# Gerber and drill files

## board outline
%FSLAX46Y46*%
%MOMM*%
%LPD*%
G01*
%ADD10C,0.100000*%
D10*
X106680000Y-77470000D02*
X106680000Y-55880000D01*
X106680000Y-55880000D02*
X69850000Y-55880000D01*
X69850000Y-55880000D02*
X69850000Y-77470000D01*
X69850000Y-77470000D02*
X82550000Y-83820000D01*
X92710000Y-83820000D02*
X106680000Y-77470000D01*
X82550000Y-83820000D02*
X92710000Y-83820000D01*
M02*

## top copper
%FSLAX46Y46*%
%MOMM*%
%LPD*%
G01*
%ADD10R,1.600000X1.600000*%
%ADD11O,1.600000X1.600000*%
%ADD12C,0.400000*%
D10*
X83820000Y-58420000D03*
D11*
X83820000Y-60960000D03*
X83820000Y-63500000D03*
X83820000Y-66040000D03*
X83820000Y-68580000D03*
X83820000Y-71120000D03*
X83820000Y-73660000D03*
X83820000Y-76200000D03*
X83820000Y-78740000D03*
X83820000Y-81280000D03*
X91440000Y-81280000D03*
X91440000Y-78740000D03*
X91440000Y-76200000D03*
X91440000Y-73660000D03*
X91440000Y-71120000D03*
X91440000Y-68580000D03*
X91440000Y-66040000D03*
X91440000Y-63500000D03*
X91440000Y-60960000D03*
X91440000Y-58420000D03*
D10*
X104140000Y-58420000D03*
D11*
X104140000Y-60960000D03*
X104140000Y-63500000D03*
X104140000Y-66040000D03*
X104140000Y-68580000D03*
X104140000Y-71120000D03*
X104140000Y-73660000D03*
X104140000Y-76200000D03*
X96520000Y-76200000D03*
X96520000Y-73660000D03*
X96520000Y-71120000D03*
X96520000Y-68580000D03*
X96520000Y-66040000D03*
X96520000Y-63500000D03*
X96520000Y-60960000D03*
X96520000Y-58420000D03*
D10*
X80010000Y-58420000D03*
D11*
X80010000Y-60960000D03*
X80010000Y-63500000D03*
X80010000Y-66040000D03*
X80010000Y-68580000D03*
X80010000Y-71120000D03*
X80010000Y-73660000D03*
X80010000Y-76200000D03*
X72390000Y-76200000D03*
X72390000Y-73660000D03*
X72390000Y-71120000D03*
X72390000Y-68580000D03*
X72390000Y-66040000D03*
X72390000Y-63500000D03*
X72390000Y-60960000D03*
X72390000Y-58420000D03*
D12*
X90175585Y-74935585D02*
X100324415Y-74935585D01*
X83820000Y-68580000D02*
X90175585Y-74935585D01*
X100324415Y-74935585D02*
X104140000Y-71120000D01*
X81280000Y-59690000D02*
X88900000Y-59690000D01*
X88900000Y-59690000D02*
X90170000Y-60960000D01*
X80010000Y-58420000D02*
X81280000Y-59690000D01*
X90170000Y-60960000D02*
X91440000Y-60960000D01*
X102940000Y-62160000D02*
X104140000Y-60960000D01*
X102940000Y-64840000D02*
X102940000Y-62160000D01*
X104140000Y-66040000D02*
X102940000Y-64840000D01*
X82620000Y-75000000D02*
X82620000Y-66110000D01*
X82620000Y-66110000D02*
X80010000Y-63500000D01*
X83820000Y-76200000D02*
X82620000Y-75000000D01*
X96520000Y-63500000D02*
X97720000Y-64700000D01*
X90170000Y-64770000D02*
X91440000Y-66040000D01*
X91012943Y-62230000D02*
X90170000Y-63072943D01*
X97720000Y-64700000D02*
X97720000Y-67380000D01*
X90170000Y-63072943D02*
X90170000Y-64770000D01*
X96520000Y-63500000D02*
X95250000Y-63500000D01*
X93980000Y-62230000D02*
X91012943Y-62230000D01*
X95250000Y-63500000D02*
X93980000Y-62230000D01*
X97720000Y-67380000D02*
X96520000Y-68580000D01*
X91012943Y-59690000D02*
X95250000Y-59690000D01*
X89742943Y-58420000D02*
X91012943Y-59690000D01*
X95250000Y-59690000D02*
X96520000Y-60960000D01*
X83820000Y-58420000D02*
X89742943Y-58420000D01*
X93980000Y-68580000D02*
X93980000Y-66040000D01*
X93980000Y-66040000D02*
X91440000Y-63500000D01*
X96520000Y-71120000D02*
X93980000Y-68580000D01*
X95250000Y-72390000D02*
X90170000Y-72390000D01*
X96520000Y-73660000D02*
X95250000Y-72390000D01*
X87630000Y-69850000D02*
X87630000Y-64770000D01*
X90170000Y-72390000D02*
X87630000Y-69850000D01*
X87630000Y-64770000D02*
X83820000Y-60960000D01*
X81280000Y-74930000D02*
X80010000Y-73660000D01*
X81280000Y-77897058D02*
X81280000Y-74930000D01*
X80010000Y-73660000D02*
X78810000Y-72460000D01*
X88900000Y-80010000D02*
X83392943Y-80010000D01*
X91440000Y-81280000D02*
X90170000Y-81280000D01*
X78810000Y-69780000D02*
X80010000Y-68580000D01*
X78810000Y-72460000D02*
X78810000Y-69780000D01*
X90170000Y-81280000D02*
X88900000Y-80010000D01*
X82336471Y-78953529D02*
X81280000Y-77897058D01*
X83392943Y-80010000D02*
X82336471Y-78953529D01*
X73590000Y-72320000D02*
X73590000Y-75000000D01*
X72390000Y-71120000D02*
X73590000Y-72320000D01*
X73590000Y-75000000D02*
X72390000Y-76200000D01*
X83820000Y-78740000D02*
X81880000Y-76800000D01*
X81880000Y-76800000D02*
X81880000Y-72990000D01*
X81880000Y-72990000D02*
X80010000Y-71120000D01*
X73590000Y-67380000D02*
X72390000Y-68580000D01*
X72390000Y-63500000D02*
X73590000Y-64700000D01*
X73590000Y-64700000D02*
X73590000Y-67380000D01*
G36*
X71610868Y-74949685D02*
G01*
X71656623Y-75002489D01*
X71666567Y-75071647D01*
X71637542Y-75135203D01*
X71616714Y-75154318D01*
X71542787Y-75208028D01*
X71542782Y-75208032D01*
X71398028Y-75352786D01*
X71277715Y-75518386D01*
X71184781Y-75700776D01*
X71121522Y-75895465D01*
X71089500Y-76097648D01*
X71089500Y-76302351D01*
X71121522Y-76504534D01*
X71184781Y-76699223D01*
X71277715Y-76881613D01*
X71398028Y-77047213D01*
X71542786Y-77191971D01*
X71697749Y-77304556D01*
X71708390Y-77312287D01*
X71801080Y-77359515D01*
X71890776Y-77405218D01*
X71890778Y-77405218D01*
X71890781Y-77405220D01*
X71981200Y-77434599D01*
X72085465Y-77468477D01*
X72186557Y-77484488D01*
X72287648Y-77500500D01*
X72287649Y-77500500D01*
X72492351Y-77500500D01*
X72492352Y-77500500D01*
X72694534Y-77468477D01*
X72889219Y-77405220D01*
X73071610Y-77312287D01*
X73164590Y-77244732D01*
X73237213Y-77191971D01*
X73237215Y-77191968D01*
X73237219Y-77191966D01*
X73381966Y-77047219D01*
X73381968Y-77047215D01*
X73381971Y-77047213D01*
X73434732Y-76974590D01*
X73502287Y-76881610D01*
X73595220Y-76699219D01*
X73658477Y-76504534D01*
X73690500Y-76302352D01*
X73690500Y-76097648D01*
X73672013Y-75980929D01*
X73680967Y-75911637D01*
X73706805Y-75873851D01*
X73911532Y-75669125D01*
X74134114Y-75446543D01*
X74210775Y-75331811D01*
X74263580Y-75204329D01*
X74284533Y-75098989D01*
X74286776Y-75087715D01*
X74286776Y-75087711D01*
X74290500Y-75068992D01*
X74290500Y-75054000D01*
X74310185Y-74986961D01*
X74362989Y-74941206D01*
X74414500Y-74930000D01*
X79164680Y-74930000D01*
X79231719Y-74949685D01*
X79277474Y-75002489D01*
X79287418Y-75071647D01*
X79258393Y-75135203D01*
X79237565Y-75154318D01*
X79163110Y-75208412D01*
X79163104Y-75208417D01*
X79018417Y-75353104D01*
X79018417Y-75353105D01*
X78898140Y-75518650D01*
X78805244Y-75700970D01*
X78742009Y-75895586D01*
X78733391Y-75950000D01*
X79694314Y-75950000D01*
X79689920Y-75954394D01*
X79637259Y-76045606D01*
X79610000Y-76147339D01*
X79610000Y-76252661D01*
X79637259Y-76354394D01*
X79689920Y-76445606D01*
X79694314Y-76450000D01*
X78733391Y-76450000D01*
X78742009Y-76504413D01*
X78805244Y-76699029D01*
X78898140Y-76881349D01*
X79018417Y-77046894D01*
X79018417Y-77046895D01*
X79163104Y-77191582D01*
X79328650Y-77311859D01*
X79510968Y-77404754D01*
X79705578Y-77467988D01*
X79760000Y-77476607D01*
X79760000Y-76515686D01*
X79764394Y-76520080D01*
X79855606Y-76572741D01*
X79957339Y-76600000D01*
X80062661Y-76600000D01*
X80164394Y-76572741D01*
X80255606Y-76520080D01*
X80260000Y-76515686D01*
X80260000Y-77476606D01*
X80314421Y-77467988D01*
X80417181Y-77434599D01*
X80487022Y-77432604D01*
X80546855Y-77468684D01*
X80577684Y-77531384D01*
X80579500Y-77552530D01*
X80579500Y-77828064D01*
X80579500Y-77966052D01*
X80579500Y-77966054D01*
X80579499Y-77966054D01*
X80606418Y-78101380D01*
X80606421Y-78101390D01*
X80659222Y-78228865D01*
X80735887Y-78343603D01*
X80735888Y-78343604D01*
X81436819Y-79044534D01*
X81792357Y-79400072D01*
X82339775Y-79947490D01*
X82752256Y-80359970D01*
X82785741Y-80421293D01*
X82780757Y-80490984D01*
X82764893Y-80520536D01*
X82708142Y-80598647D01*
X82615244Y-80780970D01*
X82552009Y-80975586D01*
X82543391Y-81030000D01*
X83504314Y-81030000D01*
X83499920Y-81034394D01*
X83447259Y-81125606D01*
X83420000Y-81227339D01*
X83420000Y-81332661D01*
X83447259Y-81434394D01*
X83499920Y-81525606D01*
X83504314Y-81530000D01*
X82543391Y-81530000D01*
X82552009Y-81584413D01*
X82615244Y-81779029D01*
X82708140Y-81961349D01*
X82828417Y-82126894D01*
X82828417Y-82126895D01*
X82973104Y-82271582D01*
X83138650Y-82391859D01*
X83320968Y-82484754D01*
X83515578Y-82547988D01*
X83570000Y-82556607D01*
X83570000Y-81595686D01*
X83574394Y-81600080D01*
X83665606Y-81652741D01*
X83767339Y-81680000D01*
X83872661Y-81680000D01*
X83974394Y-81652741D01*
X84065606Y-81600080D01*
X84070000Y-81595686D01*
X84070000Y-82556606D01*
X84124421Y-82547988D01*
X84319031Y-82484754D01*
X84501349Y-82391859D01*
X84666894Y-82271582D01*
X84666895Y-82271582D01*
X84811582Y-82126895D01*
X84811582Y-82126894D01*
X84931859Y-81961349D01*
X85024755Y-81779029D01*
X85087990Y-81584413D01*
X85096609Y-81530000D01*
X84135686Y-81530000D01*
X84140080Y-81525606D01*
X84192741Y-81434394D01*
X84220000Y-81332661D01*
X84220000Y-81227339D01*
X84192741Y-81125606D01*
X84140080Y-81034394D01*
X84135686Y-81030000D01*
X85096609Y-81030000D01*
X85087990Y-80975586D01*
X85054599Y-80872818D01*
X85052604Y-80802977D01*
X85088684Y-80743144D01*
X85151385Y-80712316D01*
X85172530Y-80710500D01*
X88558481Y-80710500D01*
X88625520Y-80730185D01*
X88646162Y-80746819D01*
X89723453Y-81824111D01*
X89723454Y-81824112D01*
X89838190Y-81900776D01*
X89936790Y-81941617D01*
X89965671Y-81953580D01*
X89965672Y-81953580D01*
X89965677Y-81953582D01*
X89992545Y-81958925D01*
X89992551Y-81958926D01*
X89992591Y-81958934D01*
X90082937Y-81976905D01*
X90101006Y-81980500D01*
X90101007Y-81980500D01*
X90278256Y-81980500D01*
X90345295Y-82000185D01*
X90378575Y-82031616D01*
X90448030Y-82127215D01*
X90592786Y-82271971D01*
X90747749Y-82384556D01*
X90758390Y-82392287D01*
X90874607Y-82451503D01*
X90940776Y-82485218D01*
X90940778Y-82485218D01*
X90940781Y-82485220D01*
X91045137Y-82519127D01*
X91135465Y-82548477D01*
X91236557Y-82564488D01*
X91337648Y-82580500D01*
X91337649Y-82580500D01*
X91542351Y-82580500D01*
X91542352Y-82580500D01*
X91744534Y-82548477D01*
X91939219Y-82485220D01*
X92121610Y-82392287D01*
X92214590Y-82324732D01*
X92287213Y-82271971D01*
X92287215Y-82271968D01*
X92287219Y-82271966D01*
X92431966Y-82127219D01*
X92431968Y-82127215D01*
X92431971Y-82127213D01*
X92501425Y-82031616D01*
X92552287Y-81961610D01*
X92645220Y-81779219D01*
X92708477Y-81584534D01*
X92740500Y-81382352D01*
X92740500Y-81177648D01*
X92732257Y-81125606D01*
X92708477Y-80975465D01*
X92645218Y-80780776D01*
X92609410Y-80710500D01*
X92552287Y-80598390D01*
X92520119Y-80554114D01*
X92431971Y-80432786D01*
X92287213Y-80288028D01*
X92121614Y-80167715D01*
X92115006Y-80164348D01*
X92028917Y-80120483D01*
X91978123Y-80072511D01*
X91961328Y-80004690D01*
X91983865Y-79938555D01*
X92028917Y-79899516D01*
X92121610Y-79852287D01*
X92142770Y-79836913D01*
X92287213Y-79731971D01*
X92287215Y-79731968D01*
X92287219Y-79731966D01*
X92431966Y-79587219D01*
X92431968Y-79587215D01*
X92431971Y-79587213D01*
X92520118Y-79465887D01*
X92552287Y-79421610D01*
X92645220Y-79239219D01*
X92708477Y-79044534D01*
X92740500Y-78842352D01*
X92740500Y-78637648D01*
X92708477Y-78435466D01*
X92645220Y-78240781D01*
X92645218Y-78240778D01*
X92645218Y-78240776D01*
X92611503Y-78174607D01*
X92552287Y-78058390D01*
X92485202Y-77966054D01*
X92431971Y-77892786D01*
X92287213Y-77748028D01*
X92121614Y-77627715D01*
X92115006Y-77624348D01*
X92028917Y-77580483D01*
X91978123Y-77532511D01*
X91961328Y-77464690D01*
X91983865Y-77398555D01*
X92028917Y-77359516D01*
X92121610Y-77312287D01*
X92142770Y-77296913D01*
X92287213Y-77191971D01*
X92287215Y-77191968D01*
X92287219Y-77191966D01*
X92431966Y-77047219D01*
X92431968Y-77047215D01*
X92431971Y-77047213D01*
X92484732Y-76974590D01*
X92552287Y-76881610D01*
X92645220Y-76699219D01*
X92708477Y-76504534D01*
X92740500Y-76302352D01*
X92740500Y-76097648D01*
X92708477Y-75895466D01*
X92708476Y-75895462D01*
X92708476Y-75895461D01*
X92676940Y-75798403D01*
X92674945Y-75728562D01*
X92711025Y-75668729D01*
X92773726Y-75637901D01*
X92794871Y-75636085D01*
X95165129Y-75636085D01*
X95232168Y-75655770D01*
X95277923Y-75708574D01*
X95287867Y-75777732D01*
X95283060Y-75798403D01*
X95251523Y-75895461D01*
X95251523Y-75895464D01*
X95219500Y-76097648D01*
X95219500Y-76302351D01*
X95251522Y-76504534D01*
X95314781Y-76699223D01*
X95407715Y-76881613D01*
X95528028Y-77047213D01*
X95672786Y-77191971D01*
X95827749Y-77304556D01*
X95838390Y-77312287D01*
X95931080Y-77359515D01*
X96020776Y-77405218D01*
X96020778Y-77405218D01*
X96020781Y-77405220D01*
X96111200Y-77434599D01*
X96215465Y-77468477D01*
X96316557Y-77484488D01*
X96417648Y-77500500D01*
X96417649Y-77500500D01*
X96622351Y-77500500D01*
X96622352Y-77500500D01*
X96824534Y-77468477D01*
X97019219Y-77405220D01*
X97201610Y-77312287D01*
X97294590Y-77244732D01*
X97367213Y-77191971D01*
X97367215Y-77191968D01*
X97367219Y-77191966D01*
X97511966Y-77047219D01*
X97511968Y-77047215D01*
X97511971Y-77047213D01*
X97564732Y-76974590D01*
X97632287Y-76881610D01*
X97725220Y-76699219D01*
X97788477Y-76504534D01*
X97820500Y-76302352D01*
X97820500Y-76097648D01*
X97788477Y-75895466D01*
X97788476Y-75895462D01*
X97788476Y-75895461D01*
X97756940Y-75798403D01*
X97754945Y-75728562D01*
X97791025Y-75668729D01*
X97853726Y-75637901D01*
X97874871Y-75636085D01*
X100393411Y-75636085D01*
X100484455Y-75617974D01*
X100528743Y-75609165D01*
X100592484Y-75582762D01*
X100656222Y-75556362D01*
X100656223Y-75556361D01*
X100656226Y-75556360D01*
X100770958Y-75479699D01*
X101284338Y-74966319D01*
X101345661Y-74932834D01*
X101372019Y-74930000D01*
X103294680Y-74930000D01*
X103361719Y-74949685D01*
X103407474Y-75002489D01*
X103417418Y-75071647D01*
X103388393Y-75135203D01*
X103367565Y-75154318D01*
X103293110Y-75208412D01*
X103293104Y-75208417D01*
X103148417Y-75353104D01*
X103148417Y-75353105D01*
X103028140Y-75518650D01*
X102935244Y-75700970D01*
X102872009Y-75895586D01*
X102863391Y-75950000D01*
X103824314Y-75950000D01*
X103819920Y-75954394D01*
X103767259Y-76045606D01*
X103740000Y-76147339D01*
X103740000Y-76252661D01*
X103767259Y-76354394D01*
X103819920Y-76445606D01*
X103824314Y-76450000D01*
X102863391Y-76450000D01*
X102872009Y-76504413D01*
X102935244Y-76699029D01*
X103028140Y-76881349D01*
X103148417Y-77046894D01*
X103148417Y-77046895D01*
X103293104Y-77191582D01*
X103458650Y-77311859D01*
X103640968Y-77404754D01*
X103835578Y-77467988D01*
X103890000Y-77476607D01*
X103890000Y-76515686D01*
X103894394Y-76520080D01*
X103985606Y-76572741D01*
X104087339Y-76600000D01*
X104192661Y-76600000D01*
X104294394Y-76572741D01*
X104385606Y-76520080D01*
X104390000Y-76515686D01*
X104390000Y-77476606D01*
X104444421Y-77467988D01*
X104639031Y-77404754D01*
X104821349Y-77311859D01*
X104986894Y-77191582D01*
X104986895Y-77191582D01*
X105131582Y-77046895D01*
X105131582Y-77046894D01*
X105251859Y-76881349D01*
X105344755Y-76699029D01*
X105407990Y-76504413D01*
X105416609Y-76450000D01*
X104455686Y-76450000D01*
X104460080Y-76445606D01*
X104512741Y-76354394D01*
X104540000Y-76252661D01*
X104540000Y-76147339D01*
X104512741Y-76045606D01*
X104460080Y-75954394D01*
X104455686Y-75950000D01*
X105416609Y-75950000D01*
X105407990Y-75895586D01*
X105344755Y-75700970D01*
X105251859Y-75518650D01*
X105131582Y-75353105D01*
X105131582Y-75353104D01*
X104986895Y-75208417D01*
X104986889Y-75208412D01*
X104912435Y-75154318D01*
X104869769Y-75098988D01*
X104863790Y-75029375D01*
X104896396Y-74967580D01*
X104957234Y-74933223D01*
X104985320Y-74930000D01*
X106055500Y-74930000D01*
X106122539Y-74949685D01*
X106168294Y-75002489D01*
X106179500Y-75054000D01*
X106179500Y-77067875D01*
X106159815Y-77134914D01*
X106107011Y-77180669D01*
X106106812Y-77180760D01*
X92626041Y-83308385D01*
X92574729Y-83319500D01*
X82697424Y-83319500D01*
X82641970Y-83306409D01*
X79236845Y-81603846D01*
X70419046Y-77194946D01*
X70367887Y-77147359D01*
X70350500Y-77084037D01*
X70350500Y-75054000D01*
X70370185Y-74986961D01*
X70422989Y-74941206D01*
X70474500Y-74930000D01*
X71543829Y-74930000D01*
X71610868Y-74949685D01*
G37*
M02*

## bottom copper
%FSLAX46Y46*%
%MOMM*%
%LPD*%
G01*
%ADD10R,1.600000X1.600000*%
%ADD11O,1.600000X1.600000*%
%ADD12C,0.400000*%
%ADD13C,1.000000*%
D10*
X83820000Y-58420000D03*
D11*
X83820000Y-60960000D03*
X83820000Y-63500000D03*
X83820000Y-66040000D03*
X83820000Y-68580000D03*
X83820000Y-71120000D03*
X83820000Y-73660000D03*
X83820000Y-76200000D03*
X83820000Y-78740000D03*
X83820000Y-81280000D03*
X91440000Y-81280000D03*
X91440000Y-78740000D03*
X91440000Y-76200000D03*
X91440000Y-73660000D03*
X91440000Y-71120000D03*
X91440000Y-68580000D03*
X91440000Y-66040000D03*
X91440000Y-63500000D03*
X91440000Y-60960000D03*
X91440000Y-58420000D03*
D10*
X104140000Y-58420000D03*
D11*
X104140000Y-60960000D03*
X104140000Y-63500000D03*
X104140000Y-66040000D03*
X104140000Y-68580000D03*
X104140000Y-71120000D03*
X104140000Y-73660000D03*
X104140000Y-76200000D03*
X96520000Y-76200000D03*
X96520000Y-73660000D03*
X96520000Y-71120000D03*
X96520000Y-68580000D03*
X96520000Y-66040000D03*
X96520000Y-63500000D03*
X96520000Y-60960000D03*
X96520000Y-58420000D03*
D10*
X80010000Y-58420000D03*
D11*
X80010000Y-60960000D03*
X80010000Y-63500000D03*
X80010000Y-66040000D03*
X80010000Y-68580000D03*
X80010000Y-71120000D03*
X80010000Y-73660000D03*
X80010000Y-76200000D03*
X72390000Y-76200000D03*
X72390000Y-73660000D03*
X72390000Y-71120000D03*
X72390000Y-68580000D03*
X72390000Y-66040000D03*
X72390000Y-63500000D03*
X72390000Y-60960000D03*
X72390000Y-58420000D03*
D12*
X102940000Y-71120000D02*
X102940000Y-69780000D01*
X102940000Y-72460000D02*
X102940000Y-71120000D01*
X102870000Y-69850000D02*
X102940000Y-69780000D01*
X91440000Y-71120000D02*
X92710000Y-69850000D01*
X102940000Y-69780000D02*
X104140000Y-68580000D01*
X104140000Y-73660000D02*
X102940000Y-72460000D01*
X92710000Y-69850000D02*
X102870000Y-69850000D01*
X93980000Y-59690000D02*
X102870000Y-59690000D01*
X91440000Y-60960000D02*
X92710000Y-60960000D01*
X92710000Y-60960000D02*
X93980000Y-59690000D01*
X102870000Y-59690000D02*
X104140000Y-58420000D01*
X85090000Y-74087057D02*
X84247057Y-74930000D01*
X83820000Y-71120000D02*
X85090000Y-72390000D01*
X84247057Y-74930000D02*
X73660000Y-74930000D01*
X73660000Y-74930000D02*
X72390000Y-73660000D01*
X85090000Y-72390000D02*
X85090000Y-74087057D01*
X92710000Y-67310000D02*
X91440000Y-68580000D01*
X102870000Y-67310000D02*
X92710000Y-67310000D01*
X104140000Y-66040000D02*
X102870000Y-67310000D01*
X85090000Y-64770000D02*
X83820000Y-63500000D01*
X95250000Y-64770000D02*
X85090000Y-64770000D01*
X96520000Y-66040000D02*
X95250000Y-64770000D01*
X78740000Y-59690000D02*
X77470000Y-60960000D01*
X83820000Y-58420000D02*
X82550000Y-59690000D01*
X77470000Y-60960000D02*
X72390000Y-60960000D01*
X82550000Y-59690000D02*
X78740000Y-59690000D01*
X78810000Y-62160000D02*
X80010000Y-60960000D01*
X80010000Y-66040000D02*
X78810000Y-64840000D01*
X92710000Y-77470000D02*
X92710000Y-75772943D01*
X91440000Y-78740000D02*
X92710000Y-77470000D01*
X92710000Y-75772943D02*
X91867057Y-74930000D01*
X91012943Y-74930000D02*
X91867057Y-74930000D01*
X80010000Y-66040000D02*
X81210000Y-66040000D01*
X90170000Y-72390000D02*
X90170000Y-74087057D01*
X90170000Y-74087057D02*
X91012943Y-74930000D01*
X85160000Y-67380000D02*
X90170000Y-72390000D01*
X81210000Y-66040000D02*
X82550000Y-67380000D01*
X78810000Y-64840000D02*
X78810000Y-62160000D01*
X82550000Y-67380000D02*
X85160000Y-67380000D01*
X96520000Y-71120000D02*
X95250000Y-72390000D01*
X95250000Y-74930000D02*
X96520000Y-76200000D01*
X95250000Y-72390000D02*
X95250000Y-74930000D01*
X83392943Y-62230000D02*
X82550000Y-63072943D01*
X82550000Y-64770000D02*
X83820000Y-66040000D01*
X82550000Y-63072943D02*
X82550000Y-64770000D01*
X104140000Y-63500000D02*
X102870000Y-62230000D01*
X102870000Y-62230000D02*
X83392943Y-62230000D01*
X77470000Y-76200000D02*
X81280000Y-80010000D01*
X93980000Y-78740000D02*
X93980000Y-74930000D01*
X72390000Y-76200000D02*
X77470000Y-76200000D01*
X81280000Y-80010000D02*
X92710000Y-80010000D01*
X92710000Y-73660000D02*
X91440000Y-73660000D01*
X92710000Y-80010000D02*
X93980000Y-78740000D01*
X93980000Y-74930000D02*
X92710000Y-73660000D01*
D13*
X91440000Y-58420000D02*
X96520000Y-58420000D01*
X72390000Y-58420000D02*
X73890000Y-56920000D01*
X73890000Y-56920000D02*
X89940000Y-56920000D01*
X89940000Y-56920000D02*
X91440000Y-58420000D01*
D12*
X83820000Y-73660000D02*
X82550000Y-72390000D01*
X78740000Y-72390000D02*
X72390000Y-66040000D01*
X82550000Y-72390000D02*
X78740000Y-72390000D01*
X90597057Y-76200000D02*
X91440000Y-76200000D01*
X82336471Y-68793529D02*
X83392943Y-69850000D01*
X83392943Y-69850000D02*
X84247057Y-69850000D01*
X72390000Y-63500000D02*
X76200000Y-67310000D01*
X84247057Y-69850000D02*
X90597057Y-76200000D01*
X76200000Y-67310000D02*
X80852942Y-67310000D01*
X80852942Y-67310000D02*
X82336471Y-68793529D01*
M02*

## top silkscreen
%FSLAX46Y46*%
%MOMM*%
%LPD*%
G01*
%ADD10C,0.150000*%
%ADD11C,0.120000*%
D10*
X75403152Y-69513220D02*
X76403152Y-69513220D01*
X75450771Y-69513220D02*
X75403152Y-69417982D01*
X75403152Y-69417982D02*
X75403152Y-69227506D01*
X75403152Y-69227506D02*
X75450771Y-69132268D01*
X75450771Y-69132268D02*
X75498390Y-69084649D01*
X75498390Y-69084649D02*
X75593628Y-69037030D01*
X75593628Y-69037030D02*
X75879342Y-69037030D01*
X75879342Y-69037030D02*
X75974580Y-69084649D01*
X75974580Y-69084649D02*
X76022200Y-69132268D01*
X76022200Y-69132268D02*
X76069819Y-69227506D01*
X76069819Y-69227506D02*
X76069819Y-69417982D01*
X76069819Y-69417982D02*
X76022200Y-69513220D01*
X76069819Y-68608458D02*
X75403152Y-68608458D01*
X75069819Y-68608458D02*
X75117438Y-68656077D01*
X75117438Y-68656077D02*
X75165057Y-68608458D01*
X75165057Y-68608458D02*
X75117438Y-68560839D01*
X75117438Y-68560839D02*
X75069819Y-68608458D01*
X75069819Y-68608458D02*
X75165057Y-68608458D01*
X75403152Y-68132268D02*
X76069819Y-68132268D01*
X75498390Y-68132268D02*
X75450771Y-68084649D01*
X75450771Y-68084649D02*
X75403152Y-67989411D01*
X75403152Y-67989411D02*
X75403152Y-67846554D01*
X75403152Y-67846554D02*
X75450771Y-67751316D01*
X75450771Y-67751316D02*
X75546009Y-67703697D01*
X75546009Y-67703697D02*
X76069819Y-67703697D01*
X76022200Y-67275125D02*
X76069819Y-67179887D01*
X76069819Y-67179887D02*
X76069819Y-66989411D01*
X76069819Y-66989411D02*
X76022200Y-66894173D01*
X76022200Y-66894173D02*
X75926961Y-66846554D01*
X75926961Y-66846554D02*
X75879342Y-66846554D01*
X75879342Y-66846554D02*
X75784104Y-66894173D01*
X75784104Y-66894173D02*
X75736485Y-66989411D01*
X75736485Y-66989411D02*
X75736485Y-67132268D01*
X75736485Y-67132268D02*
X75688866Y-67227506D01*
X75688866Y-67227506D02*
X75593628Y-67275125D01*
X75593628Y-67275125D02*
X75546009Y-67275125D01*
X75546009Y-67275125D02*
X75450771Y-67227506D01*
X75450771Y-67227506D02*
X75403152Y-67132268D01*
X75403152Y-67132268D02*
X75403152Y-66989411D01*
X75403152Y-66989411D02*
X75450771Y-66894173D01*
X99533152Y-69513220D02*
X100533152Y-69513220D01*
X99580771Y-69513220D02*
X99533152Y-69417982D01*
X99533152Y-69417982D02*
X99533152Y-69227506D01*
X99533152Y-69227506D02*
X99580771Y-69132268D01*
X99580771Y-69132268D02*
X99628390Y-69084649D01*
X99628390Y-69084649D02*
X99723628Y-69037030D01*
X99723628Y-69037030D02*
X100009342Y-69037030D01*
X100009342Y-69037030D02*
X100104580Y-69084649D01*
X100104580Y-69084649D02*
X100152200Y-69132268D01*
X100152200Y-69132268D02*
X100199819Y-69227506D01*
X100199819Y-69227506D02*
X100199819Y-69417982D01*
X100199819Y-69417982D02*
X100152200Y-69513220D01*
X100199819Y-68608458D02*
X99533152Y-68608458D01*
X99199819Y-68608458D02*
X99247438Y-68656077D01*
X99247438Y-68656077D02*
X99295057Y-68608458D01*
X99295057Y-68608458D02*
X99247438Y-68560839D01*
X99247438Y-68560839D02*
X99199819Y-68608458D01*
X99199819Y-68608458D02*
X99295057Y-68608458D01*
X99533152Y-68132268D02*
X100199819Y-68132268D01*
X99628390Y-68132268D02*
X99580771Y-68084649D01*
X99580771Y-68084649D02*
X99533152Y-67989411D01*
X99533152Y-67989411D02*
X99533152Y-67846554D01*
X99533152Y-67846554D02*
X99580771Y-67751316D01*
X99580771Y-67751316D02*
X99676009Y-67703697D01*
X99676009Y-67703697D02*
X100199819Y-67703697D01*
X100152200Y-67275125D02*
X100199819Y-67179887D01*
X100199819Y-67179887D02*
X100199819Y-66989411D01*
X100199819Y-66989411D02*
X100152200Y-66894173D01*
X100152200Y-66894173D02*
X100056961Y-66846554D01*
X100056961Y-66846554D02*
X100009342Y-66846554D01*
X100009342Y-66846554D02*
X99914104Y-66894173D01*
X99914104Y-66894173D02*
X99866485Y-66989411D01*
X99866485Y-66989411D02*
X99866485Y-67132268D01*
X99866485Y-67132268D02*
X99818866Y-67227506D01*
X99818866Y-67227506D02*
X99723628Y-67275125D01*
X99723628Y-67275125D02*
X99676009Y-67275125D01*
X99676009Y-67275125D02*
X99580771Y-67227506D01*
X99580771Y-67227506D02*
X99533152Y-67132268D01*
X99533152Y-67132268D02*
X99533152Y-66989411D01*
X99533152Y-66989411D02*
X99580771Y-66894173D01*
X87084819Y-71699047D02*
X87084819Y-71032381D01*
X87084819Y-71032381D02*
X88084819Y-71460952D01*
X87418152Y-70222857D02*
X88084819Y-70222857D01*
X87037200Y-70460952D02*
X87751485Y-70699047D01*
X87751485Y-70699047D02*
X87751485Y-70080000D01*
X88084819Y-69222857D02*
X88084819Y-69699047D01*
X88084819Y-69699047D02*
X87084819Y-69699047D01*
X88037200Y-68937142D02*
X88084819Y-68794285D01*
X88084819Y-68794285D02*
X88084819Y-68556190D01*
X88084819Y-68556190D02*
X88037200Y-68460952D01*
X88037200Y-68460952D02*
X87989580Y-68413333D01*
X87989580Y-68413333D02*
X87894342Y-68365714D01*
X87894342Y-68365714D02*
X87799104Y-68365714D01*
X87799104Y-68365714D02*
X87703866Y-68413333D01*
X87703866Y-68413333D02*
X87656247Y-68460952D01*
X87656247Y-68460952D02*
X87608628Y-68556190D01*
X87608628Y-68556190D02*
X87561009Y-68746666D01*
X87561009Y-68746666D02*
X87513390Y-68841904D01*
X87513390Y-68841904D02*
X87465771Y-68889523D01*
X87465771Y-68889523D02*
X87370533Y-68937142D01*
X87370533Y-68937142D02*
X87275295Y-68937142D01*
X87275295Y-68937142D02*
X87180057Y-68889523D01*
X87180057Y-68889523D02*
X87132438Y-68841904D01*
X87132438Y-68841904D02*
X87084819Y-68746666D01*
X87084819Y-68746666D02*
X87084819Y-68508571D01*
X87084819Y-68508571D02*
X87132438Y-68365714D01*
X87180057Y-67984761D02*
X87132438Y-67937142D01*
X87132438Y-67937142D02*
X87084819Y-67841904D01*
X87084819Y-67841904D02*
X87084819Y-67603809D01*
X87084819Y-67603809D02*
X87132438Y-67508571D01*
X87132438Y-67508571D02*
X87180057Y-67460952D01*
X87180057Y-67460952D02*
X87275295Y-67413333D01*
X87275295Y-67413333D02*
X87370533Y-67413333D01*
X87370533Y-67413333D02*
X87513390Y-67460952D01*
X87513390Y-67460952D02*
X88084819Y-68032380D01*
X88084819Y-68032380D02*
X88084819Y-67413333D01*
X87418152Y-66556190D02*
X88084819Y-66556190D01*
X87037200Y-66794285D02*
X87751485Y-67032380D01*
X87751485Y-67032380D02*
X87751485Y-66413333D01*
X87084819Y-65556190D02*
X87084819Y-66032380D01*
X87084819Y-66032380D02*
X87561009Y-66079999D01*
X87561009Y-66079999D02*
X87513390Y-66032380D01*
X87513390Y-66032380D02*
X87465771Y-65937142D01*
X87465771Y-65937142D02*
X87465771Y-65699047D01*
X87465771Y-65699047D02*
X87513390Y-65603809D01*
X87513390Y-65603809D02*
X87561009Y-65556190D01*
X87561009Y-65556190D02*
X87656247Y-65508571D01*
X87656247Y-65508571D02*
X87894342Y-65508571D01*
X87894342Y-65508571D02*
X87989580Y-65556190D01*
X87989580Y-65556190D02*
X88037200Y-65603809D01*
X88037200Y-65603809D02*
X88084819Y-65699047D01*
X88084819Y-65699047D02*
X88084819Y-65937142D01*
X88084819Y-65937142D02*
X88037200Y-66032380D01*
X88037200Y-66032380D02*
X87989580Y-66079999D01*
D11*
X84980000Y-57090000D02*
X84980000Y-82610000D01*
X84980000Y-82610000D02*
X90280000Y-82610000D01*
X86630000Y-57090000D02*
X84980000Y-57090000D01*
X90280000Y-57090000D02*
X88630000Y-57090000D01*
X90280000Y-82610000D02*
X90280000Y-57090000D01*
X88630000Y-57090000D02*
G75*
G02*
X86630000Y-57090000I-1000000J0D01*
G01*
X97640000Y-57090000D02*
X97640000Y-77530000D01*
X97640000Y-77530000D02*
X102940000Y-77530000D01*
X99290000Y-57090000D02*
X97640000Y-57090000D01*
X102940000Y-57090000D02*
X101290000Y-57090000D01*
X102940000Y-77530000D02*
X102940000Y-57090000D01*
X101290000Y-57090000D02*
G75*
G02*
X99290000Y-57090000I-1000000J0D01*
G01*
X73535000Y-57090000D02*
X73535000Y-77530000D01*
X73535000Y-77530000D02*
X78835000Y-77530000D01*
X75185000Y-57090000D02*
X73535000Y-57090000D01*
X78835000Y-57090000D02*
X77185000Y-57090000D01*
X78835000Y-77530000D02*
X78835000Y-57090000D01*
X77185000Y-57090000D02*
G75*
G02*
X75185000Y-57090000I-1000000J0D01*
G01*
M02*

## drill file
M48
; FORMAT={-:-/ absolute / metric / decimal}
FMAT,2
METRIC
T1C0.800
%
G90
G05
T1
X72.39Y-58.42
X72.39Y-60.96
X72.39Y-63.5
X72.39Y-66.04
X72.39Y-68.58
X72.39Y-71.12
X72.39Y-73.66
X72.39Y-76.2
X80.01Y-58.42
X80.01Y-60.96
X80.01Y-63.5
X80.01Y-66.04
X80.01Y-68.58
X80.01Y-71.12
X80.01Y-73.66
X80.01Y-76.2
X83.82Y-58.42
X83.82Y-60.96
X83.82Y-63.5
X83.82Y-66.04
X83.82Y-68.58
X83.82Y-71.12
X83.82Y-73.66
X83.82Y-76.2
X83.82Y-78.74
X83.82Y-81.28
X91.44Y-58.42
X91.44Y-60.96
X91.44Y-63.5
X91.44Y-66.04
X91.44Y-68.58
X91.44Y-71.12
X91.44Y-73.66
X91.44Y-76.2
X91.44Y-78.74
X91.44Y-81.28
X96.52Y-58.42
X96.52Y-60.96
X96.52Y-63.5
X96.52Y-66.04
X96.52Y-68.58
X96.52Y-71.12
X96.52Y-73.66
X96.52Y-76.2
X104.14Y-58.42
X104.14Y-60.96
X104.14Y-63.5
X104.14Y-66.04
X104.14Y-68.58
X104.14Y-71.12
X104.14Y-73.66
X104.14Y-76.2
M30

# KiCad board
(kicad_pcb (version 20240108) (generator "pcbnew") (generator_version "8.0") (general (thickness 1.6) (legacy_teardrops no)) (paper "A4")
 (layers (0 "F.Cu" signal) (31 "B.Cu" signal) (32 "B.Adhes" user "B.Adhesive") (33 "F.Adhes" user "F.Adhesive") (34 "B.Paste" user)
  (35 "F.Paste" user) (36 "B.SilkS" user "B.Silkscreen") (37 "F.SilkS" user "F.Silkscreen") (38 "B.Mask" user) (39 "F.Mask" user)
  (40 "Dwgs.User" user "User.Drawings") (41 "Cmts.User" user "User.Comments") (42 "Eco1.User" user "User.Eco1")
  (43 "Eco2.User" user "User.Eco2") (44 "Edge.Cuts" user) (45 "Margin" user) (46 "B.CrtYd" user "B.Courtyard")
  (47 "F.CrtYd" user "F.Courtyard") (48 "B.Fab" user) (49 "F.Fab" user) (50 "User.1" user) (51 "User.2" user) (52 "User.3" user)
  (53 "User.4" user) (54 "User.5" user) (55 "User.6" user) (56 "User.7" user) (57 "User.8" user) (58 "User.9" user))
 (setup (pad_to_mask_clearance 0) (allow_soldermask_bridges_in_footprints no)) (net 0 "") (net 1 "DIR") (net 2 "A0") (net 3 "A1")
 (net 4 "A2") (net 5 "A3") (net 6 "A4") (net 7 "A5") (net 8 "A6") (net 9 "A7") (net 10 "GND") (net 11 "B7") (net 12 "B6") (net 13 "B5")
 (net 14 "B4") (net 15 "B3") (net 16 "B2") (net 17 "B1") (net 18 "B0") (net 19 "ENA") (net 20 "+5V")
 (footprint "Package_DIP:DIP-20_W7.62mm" (layer "F.Cu") (at 83.82 58.42)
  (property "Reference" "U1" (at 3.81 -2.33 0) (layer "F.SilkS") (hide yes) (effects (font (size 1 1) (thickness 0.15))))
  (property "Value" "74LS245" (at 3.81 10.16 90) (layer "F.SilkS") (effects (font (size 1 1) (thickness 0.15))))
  (fp_line (start 1.16 -1.33) (end 1.16 24.19) (stroke (width 0.12) (type solid)) (layer "F.SilkS"))
  (fp_line (start 1.16 24.19) (end 6.46 24.19) (stroke (width 0.12) (type solid)) (layer "F.SilkS"))
  (fp_line (start 2.81 -1.33) (end 1.16 -1.33) (stroke (width 0.12) (type solid)) (layer "F.SilkS"))
  (fp_line (start 6.46 -1.33) (end 4.81 -1.33) (stroke (width 0.12) (type solid)) (layer "F.SilkS"))
  (fp_line (start 6.46 24.19) (end 6.46 -1.33) (stroke (width 0.12) (type solid)) (layer "F.SilkS"))
  (fp_arc (start 4.81 -1.33) (mid 3.81 -0.33) (end 2.81 -1.33) (stroke (width 0.12) (type solid)) (layer "F.SilkS"))
  (pad "1" thru_hole rect (at 0 0) (size 1.6 1.6) (drill 0.8) (layers "*.Cu" "*.Mask") (remove_unused_layers no) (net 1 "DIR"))
  (pad "2" thru_hole oval (at 0 2.54) (size 1.6 1.6) (drill 0.8) (layers "*.Cu" "*.Mask") (remove_unused_layers no) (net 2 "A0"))
  (pad "3" thru_hole oval (at 0 5.08) (size 1.6 1.6) (drill 0.8) (layers "*.Cu" "*.Mask") (remove_unused_layers no) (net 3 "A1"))
  (pad "4" thru_hole oval (at 0 7.62) (size 1.6 1.6) (drill 0.8) (layers "*.Cu" "*.Mask") (remove_unused_layers no) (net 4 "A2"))
  (pad "5" thru_hole oval (at 0 10.16) (size 1.6 1.6) (drill 0.8) (layers "*.Cu" "*.Mask") (remove_unused_layers no) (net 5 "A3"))
  (pad "6" thru_hole oval (at 0 12.7) (size 1.6 1.6) (drill 0.8) (layers "*.Cu" "*.Mask") (remove_unused_layers no) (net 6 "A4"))
  (pad "7" thru_hole oval (at 0 15.24) (size 1.6 1.6) (drill 0.8) (layers "*.Cu" "*.Mask") (remove_unused_layers no) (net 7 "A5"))
  (pad "8" thru_hole oval (at 0 17.78) (size 1.6 1.6) (drill 0.8) (layers "*.Cu" "*.Mask") (remove_unused_layers no) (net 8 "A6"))
  (pad "9" thru_hole oval (at 0 20.32) (size 1.6 1.6) (drill 0.8) (layers "*.Cu" "*.Mask") (remove_unused_layers no) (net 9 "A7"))
  (pad "10" thru_hole oval (at 0 22.86) (size 1.6 1.6) (drill 0.8) (layers "*.Cu" "*.Mask") (remove_unused_layers no) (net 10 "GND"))
  (pad "11" thru_hole oval (at 7.62 22.86) (size 1.6 1.6) (drill 0.8) (layers "*.Cu" "*.Mask") (remove_unused_layers no) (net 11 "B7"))
  (pad "12" thru_hole oval (at 7.62 20.32) (size 1.6 1.6) (drill 0.8) (layers "*.Cu" "*.Mask") (remove_unused_layers no) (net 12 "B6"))
  (pad "13" thru_hole oval (at 7.62 17.78) (size 1.6 1.6) (drill 0.8) (layers "*.Cu" "*.Mask") (remove_unused_layers no) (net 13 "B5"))
  (pad "14" thru_hole oval (at 7.62 15.24) (size 1.6 1.6) (drill 0.8) (layers "*.Cu" "*.Mask") (remove_unused_layers no) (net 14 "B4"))
  (pad "15" thru_hole oval (at 7.62 12.7) (size 1.6 1.6) (drill 0.8) (layers "*.Cu" "*.Mask") (remove_unused_layers no) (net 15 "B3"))
  (pad "16" thru_hole oval (at 7.62 10.16) (size 1.6 1.6) (drill 0.8) (layers "*.Cu" "*.Mask") (remove_unused_layers no) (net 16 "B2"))
  (pad "17" thru_hole oval (at 7.62 7.62) (size 1.6 1.6) (drill 0.8) (layers "*.Cu" "*.Mask") (remove_unused_layers no) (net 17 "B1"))
  (pad "18" thru_hole oval (at 7.62 5.08) (size 1.6 1.6) (drill 0.8) (layers "*.Cu" "*.Mask") (remove_unused_layers no) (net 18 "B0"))
  (pad "19" thru_hole oval (at 7.62 2.54) (size 1.6 1.6) (drill 0.8) (layers "*.Cu" "*.Mask") (remove_unused_layers no) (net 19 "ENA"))
  (pad "20" thru_hole oval (at 7.62 0) (size 1.6 1.6) (drill 0.8) (layers "*.Cu" "*.Mask") (remove_unused_layers no) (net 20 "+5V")))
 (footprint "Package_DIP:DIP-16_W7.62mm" (layer "B.Cu") (at 104.14 58.42 180)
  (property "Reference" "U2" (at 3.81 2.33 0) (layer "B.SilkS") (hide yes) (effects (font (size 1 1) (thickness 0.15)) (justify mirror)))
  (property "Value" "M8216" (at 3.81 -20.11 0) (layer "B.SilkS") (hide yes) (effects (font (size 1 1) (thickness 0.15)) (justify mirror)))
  (fp_line (start 6.5 1.33) (end 6.5 -19.11) (stroke (width 0.12) (type solid)) (layer "F.SilkS"))
  (fp_line (start 6.5 -19.11) (end 1.2 -19.11) (stroke (width 0.12) (type solid)) (layer "F.SilkS"))
  (fp_line (start 4.85 1.33) (end 6.5 1.33) (stroke (width 0.12) (type solid)) (layer "F.SilkS"))
  (fp_line (start 1.2 1.33) (end 2.85 1.33) (stroke (width 0.12) (type solid)) (layer "F.SilkS"))
  (fp_line (start 1.2 -19.11) (end 1.2 1.33) (stroke (width 0.12) (type solid)) (layer "F.SilkS"))
  (fp_arc (start 2.85 1.33) (mid 3.85 0.33) (end 4.85 1.33) (stroke (width 0.12) (type solid)) (layer "F.SilkS"))
  (pad "1" thru_hole rect (at 0 0 180) (size 1.6 1.6) (drill 0.8) (layers "*.Cu" "*.Mask") (remove_unused_layers no) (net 19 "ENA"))
  (pad "2" thru_hole oval (at 0 -2.54 180) (size 1.6 1.6) (drill 0.8) (layers "*.Cu" "*.Mask") (remove_unused_layers no) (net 16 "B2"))
  (pad "3" thru_hole oval (at 0 -5.08 180) (size 1.6 1.6) (drill 0.8) (layers "*.Cu" "*.Mask") (remove_unused_layers no) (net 4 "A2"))
  (pad "4" thru_hole oval (at 0 -7.62 180) (size 1.6 1.6) (drill 0.8) (layers "*.Cu" "*.Mask") (remove_unused_layers no) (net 16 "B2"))
  (pad "5" thru_hole oval (at 0 -10.16 180) (size 1.6 1.6) (drill 0.8) (layers "*.Cu" "*.Mask") (remove_unused_layers no) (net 15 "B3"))
  (pad "6" thru_hole oval (at 0 -12.7 180) (size 1.6 1.6) (drill 0.8) (layers "*.Cu" "*.Mask") (remove_unused_layers no) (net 5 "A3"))
  (pad "7" thru_hole oval (at 0 -15.24 180) (size 1.6 1.6) (drill 0.8) (layers "*.Cu" "*.Mask") (remove_unused_layers no) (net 15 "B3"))
  (pad "8" thru_hole oval (at 0 -17.78 180) (size 1.6 1.6) (drill 0.8) (layers "*.Cu" "*.Mask") (remove_unused_layers no) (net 10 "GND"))
  (pad "9" thru_hole oval (at 7.62 -17.78 180) (size 1.6 1.6) (drill 0.8) (layers "*.Cu" "*.Mask") (remove_unused_layers no) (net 18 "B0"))
  (pad "10" thru_hole oval (at 7.62 -15.24 180) (size 1.6 1.6) (drill 0.8) (layers "*.Cu" "*.Mask") (remove_unused_layers no) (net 2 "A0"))
  (pad "11" thru_hole oval (at 7.62 -12.7 180) (size 1.6 1.6) (drill 0.8) (layers "*.Cu" "*.Mask") (remove_unused_layers no) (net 18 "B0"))
  (pad "12" thru_hole oval (at 7.62 -10.16 180) (size 1.6 1.6) (drill 0.8) (layers "*.Cu" "*.Mask") (remove_unused_layers no) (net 17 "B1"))
  (pad "13" thru_hole oval (at 7.62 -7.62 180) (size 1.6 1.6) (drill 0.8) (layers "*.Cu" "*.Mask") (remove_unused_layers no) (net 3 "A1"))
  (pad "14" thru_hole oval (at 7.62 -5.08 180) (size 1.6 1.6) (drill 0.8) (layers "*.Cu" "*.Mask") (remove_unused_layers no) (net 17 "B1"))
  (pad "15" thru_hole oval (at 7.62 -2.54 180) (size 1.6 1.6) (drill 0.8) (layers "*.Cu" "*.Mask") (remove_unused_layers no) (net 1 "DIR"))
  (pad "16" thru_hole oval (at 7.62 0 180) (size 1.6 1.6) (drill 0.8) (layers "*.Cu" "*.Mask") (remove_unused_layers no) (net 20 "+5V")))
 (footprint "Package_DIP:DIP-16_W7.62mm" (layer "B.Cu") (at 80.01 58.42 180)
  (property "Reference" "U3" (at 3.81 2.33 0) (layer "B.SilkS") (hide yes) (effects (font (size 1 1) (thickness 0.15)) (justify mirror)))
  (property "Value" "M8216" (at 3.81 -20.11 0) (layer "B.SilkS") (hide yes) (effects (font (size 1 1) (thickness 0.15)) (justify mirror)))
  (fp_line (start 6.475 1.33) (end 6.475 -19.11) (stroke (width 0.12) (type solid)) (layer "F.SilkS"))
  (fp_line (start 6.475 -19.11) (end 1.175 -19.11) (stroke (width 0.12) (type solid)) (layer "F.SilkS"))
  (fp_line (start 4.825 1.33) (end 6.475 1.33) (stroke (width 0.12) (type solid)) (layer "F.SilkS"))
  (fp_line (start 1.175 1.33) (end 2.825 1.33) (stroke (width 0.12) (type solid)) (layer "F.SilkS"))
  (fp_line (start 1.175 -19.11) (end 1.175 1.33) (stroke (width 0.12) (type solid)) (layer "F.SilkS"))
  (fp_arc (start 2.825 1.33) (mid 3.825 0.33) (end 4.825 1.33) (stroke (width 0.12) (type solid)) (layer "F.SilkS"))
  (pad "1" thru_hole rect (at 0 0 180) (size 1.6 1.6) (drill 0.8) (layers "*.Cu" "*.Mask") (remove_unused_layers no) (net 19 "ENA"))
  (pad "2" thru_hole oval (at 0 -2.54 180) (size 1.6 1.6) (drill 0.8) (layers "*.Cu" "*.Mask") (remove_unused_layers no) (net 12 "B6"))
  (pad "3" thru_hole oval (at 0 -5.08 180) (size 1.6 1.6) (drill 0.8) (layers "*.Cu" "*.Mask") (remove_unused_layers no) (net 8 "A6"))
  (pad "4" thru_hole oval (at 0 -7.62 180) (size 1.6 1.6) (drill 0.8) (layers "*.Cu" "*.Mask") (remove_unused_layers no) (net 12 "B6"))
  (pad "5" thru_hole oval (at 0 -10.16 180) (size 1.6 1.6) (drill 0.8) (layers "*.Cu" "*.Mask") (remove_unused_layers no) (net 11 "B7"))
  (pad "6" thru_hole oval (at 0 -12.7 180) (size 1.6 1.6) (drill 0.8) (layers "*.Cu" "*.Mask") (remove_unused_layers no) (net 9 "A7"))
  (pad "7" thru_hole oval (at 0 -15.24 180) (size 1.6 1.6) (drill 0.8) (layers "*.Cu" "*.Mask") (remove_unused_layers no) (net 11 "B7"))
  (pad "8" thru_hole oval (at 0 -17.78 180) (size 1.6 1.6) (drill 0.8) (layers "*.Cu" "*.Mask") (remove_unused_layers no) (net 10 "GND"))
  (pad "9" thru_hole oval (at 7.62 -17.78 180) (size 1.6 1.6) (drill 0.8) (layers "*.Cu" "*.Mask") (remove_unused_layers no) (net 14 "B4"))
  (pad "10" thru_hole oval (at 7.62 -15.24 180) (size 1.6 1.6) (drill 0.8) (layers "*.Cu" "*.Mask") (remove_unused_layers no) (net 6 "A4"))
  (pad "11" thru_hole oval (at 7.62 -12.7 180) (size 1.6 1.6) (drill 0.8) (layers "*.Cu" "*.Mask") (remove_unused_layers no) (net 14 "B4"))
  (pad "12" thru_hole oval (at 7.62 -10.16 180) (size 1.6 1.6) (drill 0.8) (layers "*.Cu" "*.Mask") (remove_unused_layers no) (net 13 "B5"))
  (pad "13" thru_hole oval (at 7.62 -7.62 180) (size 1.6 1.6) (drill 0.8) (layers "*.Cu" "*.Mask") (remove_unused_layers no) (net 7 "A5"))
  (pad "14" thru_hole oval (at 7.62 -5.08 180) (size 1.6 1.6) (drill 0.8) (layers "*.Cu" "*.Mask") (remove_unused_layers no) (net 13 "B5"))
  (pad "15" thru_hole oval (at 7.62 -2.54 180) (size 1.6 1.6) (drill 0.8) (layers "*.Cu" "*.Mask") (remove_unused_layers no) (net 1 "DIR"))
  (pad "16" thru_hole oval (at 7.62 0 180) (size 1.6 1.6) (drill 0.8) (layers "*.Cu" "*.Mask") (remove_unused_layers no) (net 20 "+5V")))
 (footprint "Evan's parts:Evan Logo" (layer "B.Cu") (at 87.63 59.69 -90)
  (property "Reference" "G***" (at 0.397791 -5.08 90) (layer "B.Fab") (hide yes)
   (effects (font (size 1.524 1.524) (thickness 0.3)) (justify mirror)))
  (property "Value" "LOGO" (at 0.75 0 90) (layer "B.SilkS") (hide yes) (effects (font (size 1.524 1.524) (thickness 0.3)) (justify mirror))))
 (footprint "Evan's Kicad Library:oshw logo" (layer "B.Cu") (at 100.33 67.31 -90)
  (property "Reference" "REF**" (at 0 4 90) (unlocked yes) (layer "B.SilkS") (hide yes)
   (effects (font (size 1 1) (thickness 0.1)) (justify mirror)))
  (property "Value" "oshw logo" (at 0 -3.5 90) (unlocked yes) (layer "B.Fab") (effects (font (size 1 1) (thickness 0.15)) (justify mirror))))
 (gr_line (start 106.68 77.47) (end 106.68 55.88) (stroke (width 0.1) (type default)) (layer "Edge.Cuts"))
 (gr_line (start 106.68 55.88) (end 69.85 55.88) (stroke (width 0.1) (type default)) (layer "Edge.Cuts"))
 (gr_line (start 69.85 55.88) (end 69.85 77.47) (stroke (width 0.1) (type default)) (layer "Edge.Cuts"))
 (gr_line (start 69.85 77.47) (end 82.55 83.82) (stroke (width 0.1) (type default)) (layer "Edge.Cuts"))
 (gr_line (start 92.71 83.82) (end 106.68 77.47) (stroke (width 0.1) (type default)) (layer "Edge.Cuts"))
 (gr_line (start 82.55 83.82) (end 92.71 83.82) (stroke (width 0.1) (type default)) (layer "Edge.Cuts"))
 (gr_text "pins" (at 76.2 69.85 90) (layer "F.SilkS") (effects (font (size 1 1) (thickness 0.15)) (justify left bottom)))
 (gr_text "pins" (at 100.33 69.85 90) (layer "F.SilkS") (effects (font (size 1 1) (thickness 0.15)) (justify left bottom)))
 (segment (start 90.175585 74.935585) (end 100.324415 74.935585) (width 0.4) (layer "F.Cu") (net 5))
 (segment (start 83.82 68.58) (end 90.175585 74.935585) (width 0.4) (layer "F.Cu") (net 5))
 (segment (start 100.324415 74.935585) (end 104.14 71.12) (width 0.4) (layer "F.Cu") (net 5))
 (segment (start 102.94 71.12) (end 102.94 69.78) (width 0.4) (layer "B.Cu") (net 15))
 (segment (start 102.94 72.46) (end 102.94 71.12) (width 0.4) (layer "B.Cu") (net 15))
 (segment (start 102.87 69.85) (end 102.94 69.78) (width 0.4) (layer "B.Cu") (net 15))
 (segment (start 91.44 71.12) (end 92.71 69.85) (width 0.4) (layer "B.Cu") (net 15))
 (segment (start 102.94 69.78) (end 104.14 68.58) (width 0.4) (layer "B.Cu") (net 15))
 (segment (start 104.14 73.66) (end 102.94 72.46) (width 0.4) (layer "B.Cu") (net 15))
 (segment (start 92.71 69.85) (end 102.87 69.85) (width 0.4) (layer "B.Cu") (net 15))
 (segment (start 81.28 59.69) (end 88.9 59.69) (width 0.4) (layer "F.Cu") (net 19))
 (segment (start 88.9 59.69) (end 90.17 60.96) (width 0.4) (layer "F.Cu") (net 19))
 (segment (start 80.01 58.42) (end 81.28 59.69) (width 0.4) (layer "F.Cu") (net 19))
 (segment (start 90.17 60.96) (end 91.44 60.96) (width 0.4) (layer "F.Cu") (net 19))
 (segment (start 93.98 59.69) (end 102.87 59.69) (width 0.4) (layer "B.Cu") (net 19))
 (segment (start 91.44 60.96) (end 92.71 60.96) (width 0.4) (layer "B.Cu") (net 19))
 (segment (start 92.71 60.96) (end 93.98 59.69) (width 0.4) (layer "B.Cu") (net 19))
 (segment (start 102.87 59.69) (end 104.14 58.42) (width 0.4) (layer "B.Cu") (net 19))
 (segment (start 85.09 74.087057) (end 84.247057 74.93) (width 0.4) (layer "B.Cu") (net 6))
 (segment (start 83.82 71.12) (end 85.09 72.39) (width 0.4) (layer "B.Cu") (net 6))
 (segment (start 84.247057 74.93) (end 73.66 74.93) (width 0.4) (layer "B.Cu") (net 6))
 (segment (start 73.66 74.93) (end 72.39 73.66) (width 0.4) (layer "B.Cu") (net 6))
 (segment (start 85.09 72.39) (end 85.09 74.087057) (width 0.4) (layer "B.Cu") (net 6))
 (segment (start 102.94 62.16) (end 104.14 60.96) (width 0.4) (layer "F.Cu") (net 16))
 (segment (start 102.94 64.84) (end 102.94 62.16) (width 0.4) (layer "F.Cu") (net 16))
 (segment (start 104.14 66.04) (end 102.94 64.84) (width 0.4) (layer "F.Cu") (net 16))
 (segment (start 92.71 67.31) (end 91.44 68.58) (width 0.4) (layer "B.Cu") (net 16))
 (segment (start 102.87 67.31) (end 92.71 67.31) (width 0.4) (layer "B.Cu") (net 16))
 (segment (start 104.14 66.04) (end 102.87 67.31) (width 0.4) (layer "B.Cu") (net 16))
 (segment (start 82.62 75) (end 82.62 66.11) (width 0.4) (layer "F.Cu") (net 8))
 (segment (start 82.62 66.11) (end 80.01 63.5) (width 0.4) (layer "F.Cu") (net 8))
 (segment (start 83.82 76.2) (end 82.62 75) (width 0.4) (layer "F.Cu") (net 8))
 (segment (start 96.52 63.5) (end 97.72 64.7) (width 0.4) (layer "F.Cu") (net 17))
 (segment (start 90.17 64.77) (end 91.44 66.04) (width 0.4) (layer "F.Cu") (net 17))
 (segment (start 91.012943 62.23) (end 90.17 63.072943) (width 0.4) (layer "F.Cu") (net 17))
 (segment (start 97.72 64.7) (end 97.72 67.38) (width 0.4) (layer "F.Cu") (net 17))
 (segment (start 90.17 63.072943) (end 90.17 64.77) (width 0.4) (layer "F.Cu") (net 17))
 (segment (start 96.52 63.5) (end 95.25 63.5) (width 0.4) (layer "F.Cu") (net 17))
 (segment (start 93.98 62.23) (end 91.012943 62.23) (width 0.4) (layer "F.Cu") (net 17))
 (segment (start 95.25 63.5) (end 93.98 62.23) (width 0.4) (layer "F.Cu") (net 17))
 (segment (start 97.72 67.38) (end 96.52 68.58) (width 0.4) (layer "F.Cu") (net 17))
 (segment (start 85.09 64.77) (end 83.82 63.5) (width 0.4) (layer "B.Cu") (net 3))
 (segment (start 95.25 64.77) (end 85.09 64.77) (width 0.4) (layer "B.Cu") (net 3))
 (segment (start 96.52 66.04) (end 95.25 64.77) (width 0.4) (layer "B.Cu") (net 3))
 (segment (start 91.012943 59.69) (end 95.25 59.69) (width 0.4) (layer "F.Cu") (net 1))
 (segment (start 89.742943 58.42) (end 91.012943 59.69) (width 0.4) (layer "F.Cu") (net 1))
 (segment (start 95.25 59.69) (end 96.52 60.96) (width 0.4) (layer "F.Cu") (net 1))
 (segment (start 83.82 58.42) (end 89.742943 58.42) (width 0.4) (layer "F.Cu") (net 1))
 (segment (start 78.74 59.69) (end 77.47 60.96) (width 0.4) (layer "B.Cu") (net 1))
 (segment (start 83.82 58.42) (end 82.55 59.69) (width 0.4) (layer "B.Cu") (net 1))
 (segment (start 77.47 60.96) (end 72.39 60.96) (width 0.4) (layer "B.Cu") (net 1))
 (segment (start 82.55 59.69) (end 78.74 59.69) (width 0.4) (layer "B.Cu") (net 1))
 (segment (start 78.81 62.16) (end 80.01 60.96) (width 0.4) (layer "B.Cu") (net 12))
 (segment (start 80.01 66.04) (end 78.81 64.84) (width 0.4) (layer "B.Cu") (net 12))
 (segment (start 92.71 77.47) (end 92.71 75.772943) (width 0.4) (layer "B.Cu") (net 12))
 (segment (start 91.44 78.74) (end 92.71 77.47) (width 0.4) (layer "B.Cu") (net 12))
 (segment (start 92.71 75.772943) (end 91.867057 74.93) (width 0.4) (layer "B.Cu") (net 12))
 (segment (start 91.012943 74.93) (end 91.867057 74.93) (width 0.4) (layer "B.Cu") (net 12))
 (segment (start 80.01 66.04) (end 81.21 66.04) (width 0.4) (layer "B.Cu") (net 12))
 (segment (start 90.17 72.39) (end 90.17 74.087057) (width 0.4) (layer "B.Cu") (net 12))
 (segment (start 90.17 74.087057) (end 91.012943 74.93) (width 0.4) (layer "B.Cu") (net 12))
 (segment (start 85.16 67.38) (end 90.17 72.39) (width 0.4) (layer "B.Cu") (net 12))
 (segment (start 81.21 66.04) (end 82.55 67.38) (width 0.4) (layer "B.Cu") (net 12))
 (segment (start 78.81 64.84) (end 78.81 62.16) (width 0.4) (layer "B.Cu") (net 12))
 (segment (start 82.55 67.38) (end 85.16 67.38) (width 0.4) (layer "B.Cu") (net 12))
 (segment (start 93.98 68.58) (end 93.98 66.04) (width 0.4) (layer "F.Cu") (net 18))
 (segment (start 93.98 66.04) (end 91.44 63.5) (width 0.4) (layer "F.Cu") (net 18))
 (segment (start 96.52 71.12) (end 93.98 68.58) (width 0.4) (layer "F.Cu") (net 18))
 (segment (start 96.52 71.12) (end 95.25 72.39) (width 0.4) (layer "B.Cu") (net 18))
 (segment (start 95.25 74.93) (end 96.52 76.2) (width 0.4) (layer "B.Cu") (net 18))
 (segment (start 95.25 72.39) (end 95.25 74.93) (width 0.4) (layer "B.Cu") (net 18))
 (segment (start 83.392943 62.23) (end 82.55 63.072943) (width 0.4) (layer "B.Cu") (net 4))
 (segment (start 82.55 64.77) (end 83.82 66.04) (width 0.4) (layer "B.Cu") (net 4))
 (segment (start 82.55 63.072943) (end 82.55 64.77) (width 0.4) (layer "B.Cu") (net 4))
 (segment (start 104.14 63.5) (end 102.87 62.23) (width 0.4) (layer "B.Cu") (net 4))
 (segment (start 102.87 62.23) (end 83.392943 62.23) (width 0.4) (layer "B.Cu") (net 4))
 (segment (start 95.25 72.39) (end 90.17 72.39) (width 0.4) (layer "F.Cu") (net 2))
 (segment (start 96.52 73.66) (end 95.25 72.39) (width 0.4) (layer "F.Cu") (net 2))
 (segment (start 87.63 69.85) (end 87.63 64.77) (width 0.4) (layer "F.Cu") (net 2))
 (segment (start 90.17 72.39) (end 87.63 69.85) (width 0.4) (layer "F.Cu") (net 2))
 (segment (start 87.63 64.77) (end 83.82 60.96) (width 0.4) (layer "F.Cu") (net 2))
 (segment (start 81.28 74.93) (end 80.01 73.66) (width 0.4) (layer "F.Cu") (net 11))
 (segment (start 81.28 77.897058) (end 81.28 74.93) (width 0.4) (layer "F.Cu") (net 11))
 (segment (start 80.01 73.66) (end 78.81 72.46) (width 0.4) (layer "F.Cu") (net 11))
 (segment (start 88.9 80.01) (end 83.392943 80.01) (width 0.4) (layer "F.Cu") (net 11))
 (segment (start 91.44 81.28) (end 90.17 81.28) (width 0.4) (layer "F.Cu") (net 11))
 (segment (start 78.81 69.78) (end 80.01 68.58) (width 0.4) (layer "F.Cu") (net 11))
 (segment (start 78.81 72.46) (end 78.81 69.78) (width 0.4) (layer "F.Cu") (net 11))
 (segment (start 90.17 81.28) (end 88.9 80.01) (width 0.4) (layer "F.Cu") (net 11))
 (segment (start 82.336471 78.953529) (end 81.28 77.897058) (width 0.4) (layer "F.Cu") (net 11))
 (segment (start 83.392943 80.01) (end 82.336471 78.953529) (width 0.4) (layer "F.Cu") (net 11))
 (segment (start 73.59 72.32) (end 73.59 75) (width 0.4) (layer "F.Cu") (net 14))
 (segment (start 72.39 71.12) (end 73.59 72.32) (width 0.4) (layer "F.Cu") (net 14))
 (segment (start 73.59 75) (end 72.39 76.2) (width 0.4) (layer "F.Cu") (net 14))
 (segment (start 77.47 76.2) (end 81.28 80.01) (width 0.4) (layer "B.Cu") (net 14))
 (segment (start 93.98 78.74) (end 93.98 74.93) (width 0.4) (layer "B.Cu") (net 14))
 (segment (start 72.39 76.2) (end 77.47 76.2) (width 0.4) (layer "B.Cu") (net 14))
 (segment (start 81.28 80.01) (end 92.71 80.01) (width 0.4) (layer "B.Cu") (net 14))
 (segment (start 92.71 73.66) (end 91.44 73.66) (width 0.4) (layer "B.Cu") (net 14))
 (segment (start 92.71 80.01) (end 93.98 78.74) (width 0.4) (layer "B.Cu") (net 14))
 (segment (start 93.98 74.93) (end 92.71 73.66) (width 0.4) (layer "B.Cu") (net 14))
 (segment (start 91.44 58.42) (end 96.52 58.42) (width 1) (layer "B.Cu") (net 20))
 (segment (start 72.39 58.42) (end 73.89 56.92) (width 1) (layer "B.Cu") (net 20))
 (segment (start 73.89 56.92) (end 89.94 56.92) (width 1) (layer "B.Cu") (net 20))
 (segment (start 89.94 56.92) (end 91.44 58.42) (width 1) (layer "B.Cu") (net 20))
 (segment (start 83.82 78.74) (end 81.88 76.8) (width 0.4) (layer "F.Cu") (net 9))
 (segment (start 81.88 76.8) (end 81.88 72.99) (width 0.4) (layer "F.Cu") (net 9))
 (segment (start 81.88 72.99) (end 80.01 71.12) (width 0.4) (layer "F.Cu") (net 9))
 (segment (start 83.82 73.66) (end 82.55 72.39) (width 0.4) (layer "B.Cu") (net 7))
 (segment (start 78.74 72.39) (end 72.39 66.04) (width 0.4) (layer "B.Cu") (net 7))
 (segment (start 82.55 72.39) (end 78.74 72.39) (width 0.4) (layer "B.Cu") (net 7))
 (segment (start 73.59 67.38) (end 72.39 68.58) (width 0.4) (layer "F.Cu") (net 13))
 (segment (start 72.39 63.5) (end 73.59 64.7) (width 0.4) (layer "F.Cu") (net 13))
 (segment (start 73.59 64.7) (end 73.59 67.38) (width 0.4) (layer "F.Cu") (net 13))
 (segment (start 90.597057 76.2) (end 91.44 76.2) (width 0.4) (layer "B.Cu") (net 13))
 (segment (start 82.336471 68.793529) (end 83.392943 69.85) (width 0.4) (layer "B.Cu") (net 13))
 (segment (start 83.392943 69.85) (end 84.247057 69.85) (width 0.4) (layer "B.Cu") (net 13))
 (segment (start 72.39 63.5) (end 76.2 67.31) (width 0.4) (layer "B.Cu") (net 13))
 (segment (start 84.247057 69.85) (end 90.597057 76.2) (width 0.4) (layer "B.Cu") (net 13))
 (segment (start 76.2 67.31) (end 80.852942 67.31) (width 0.4) (layer "B.Cu") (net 13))
 (segment (start 80.852942 67.31) (end 82.336471 68.793529) (width 0.4) (layer "B.Cu") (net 13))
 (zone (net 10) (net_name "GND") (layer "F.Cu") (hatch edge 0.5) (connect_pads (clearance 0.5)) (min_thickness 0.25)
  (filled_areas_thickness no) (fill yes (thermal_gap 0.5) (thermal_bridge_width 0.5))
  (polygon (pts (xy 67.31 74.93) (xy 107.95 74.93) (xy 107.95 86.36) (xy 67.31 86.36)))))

